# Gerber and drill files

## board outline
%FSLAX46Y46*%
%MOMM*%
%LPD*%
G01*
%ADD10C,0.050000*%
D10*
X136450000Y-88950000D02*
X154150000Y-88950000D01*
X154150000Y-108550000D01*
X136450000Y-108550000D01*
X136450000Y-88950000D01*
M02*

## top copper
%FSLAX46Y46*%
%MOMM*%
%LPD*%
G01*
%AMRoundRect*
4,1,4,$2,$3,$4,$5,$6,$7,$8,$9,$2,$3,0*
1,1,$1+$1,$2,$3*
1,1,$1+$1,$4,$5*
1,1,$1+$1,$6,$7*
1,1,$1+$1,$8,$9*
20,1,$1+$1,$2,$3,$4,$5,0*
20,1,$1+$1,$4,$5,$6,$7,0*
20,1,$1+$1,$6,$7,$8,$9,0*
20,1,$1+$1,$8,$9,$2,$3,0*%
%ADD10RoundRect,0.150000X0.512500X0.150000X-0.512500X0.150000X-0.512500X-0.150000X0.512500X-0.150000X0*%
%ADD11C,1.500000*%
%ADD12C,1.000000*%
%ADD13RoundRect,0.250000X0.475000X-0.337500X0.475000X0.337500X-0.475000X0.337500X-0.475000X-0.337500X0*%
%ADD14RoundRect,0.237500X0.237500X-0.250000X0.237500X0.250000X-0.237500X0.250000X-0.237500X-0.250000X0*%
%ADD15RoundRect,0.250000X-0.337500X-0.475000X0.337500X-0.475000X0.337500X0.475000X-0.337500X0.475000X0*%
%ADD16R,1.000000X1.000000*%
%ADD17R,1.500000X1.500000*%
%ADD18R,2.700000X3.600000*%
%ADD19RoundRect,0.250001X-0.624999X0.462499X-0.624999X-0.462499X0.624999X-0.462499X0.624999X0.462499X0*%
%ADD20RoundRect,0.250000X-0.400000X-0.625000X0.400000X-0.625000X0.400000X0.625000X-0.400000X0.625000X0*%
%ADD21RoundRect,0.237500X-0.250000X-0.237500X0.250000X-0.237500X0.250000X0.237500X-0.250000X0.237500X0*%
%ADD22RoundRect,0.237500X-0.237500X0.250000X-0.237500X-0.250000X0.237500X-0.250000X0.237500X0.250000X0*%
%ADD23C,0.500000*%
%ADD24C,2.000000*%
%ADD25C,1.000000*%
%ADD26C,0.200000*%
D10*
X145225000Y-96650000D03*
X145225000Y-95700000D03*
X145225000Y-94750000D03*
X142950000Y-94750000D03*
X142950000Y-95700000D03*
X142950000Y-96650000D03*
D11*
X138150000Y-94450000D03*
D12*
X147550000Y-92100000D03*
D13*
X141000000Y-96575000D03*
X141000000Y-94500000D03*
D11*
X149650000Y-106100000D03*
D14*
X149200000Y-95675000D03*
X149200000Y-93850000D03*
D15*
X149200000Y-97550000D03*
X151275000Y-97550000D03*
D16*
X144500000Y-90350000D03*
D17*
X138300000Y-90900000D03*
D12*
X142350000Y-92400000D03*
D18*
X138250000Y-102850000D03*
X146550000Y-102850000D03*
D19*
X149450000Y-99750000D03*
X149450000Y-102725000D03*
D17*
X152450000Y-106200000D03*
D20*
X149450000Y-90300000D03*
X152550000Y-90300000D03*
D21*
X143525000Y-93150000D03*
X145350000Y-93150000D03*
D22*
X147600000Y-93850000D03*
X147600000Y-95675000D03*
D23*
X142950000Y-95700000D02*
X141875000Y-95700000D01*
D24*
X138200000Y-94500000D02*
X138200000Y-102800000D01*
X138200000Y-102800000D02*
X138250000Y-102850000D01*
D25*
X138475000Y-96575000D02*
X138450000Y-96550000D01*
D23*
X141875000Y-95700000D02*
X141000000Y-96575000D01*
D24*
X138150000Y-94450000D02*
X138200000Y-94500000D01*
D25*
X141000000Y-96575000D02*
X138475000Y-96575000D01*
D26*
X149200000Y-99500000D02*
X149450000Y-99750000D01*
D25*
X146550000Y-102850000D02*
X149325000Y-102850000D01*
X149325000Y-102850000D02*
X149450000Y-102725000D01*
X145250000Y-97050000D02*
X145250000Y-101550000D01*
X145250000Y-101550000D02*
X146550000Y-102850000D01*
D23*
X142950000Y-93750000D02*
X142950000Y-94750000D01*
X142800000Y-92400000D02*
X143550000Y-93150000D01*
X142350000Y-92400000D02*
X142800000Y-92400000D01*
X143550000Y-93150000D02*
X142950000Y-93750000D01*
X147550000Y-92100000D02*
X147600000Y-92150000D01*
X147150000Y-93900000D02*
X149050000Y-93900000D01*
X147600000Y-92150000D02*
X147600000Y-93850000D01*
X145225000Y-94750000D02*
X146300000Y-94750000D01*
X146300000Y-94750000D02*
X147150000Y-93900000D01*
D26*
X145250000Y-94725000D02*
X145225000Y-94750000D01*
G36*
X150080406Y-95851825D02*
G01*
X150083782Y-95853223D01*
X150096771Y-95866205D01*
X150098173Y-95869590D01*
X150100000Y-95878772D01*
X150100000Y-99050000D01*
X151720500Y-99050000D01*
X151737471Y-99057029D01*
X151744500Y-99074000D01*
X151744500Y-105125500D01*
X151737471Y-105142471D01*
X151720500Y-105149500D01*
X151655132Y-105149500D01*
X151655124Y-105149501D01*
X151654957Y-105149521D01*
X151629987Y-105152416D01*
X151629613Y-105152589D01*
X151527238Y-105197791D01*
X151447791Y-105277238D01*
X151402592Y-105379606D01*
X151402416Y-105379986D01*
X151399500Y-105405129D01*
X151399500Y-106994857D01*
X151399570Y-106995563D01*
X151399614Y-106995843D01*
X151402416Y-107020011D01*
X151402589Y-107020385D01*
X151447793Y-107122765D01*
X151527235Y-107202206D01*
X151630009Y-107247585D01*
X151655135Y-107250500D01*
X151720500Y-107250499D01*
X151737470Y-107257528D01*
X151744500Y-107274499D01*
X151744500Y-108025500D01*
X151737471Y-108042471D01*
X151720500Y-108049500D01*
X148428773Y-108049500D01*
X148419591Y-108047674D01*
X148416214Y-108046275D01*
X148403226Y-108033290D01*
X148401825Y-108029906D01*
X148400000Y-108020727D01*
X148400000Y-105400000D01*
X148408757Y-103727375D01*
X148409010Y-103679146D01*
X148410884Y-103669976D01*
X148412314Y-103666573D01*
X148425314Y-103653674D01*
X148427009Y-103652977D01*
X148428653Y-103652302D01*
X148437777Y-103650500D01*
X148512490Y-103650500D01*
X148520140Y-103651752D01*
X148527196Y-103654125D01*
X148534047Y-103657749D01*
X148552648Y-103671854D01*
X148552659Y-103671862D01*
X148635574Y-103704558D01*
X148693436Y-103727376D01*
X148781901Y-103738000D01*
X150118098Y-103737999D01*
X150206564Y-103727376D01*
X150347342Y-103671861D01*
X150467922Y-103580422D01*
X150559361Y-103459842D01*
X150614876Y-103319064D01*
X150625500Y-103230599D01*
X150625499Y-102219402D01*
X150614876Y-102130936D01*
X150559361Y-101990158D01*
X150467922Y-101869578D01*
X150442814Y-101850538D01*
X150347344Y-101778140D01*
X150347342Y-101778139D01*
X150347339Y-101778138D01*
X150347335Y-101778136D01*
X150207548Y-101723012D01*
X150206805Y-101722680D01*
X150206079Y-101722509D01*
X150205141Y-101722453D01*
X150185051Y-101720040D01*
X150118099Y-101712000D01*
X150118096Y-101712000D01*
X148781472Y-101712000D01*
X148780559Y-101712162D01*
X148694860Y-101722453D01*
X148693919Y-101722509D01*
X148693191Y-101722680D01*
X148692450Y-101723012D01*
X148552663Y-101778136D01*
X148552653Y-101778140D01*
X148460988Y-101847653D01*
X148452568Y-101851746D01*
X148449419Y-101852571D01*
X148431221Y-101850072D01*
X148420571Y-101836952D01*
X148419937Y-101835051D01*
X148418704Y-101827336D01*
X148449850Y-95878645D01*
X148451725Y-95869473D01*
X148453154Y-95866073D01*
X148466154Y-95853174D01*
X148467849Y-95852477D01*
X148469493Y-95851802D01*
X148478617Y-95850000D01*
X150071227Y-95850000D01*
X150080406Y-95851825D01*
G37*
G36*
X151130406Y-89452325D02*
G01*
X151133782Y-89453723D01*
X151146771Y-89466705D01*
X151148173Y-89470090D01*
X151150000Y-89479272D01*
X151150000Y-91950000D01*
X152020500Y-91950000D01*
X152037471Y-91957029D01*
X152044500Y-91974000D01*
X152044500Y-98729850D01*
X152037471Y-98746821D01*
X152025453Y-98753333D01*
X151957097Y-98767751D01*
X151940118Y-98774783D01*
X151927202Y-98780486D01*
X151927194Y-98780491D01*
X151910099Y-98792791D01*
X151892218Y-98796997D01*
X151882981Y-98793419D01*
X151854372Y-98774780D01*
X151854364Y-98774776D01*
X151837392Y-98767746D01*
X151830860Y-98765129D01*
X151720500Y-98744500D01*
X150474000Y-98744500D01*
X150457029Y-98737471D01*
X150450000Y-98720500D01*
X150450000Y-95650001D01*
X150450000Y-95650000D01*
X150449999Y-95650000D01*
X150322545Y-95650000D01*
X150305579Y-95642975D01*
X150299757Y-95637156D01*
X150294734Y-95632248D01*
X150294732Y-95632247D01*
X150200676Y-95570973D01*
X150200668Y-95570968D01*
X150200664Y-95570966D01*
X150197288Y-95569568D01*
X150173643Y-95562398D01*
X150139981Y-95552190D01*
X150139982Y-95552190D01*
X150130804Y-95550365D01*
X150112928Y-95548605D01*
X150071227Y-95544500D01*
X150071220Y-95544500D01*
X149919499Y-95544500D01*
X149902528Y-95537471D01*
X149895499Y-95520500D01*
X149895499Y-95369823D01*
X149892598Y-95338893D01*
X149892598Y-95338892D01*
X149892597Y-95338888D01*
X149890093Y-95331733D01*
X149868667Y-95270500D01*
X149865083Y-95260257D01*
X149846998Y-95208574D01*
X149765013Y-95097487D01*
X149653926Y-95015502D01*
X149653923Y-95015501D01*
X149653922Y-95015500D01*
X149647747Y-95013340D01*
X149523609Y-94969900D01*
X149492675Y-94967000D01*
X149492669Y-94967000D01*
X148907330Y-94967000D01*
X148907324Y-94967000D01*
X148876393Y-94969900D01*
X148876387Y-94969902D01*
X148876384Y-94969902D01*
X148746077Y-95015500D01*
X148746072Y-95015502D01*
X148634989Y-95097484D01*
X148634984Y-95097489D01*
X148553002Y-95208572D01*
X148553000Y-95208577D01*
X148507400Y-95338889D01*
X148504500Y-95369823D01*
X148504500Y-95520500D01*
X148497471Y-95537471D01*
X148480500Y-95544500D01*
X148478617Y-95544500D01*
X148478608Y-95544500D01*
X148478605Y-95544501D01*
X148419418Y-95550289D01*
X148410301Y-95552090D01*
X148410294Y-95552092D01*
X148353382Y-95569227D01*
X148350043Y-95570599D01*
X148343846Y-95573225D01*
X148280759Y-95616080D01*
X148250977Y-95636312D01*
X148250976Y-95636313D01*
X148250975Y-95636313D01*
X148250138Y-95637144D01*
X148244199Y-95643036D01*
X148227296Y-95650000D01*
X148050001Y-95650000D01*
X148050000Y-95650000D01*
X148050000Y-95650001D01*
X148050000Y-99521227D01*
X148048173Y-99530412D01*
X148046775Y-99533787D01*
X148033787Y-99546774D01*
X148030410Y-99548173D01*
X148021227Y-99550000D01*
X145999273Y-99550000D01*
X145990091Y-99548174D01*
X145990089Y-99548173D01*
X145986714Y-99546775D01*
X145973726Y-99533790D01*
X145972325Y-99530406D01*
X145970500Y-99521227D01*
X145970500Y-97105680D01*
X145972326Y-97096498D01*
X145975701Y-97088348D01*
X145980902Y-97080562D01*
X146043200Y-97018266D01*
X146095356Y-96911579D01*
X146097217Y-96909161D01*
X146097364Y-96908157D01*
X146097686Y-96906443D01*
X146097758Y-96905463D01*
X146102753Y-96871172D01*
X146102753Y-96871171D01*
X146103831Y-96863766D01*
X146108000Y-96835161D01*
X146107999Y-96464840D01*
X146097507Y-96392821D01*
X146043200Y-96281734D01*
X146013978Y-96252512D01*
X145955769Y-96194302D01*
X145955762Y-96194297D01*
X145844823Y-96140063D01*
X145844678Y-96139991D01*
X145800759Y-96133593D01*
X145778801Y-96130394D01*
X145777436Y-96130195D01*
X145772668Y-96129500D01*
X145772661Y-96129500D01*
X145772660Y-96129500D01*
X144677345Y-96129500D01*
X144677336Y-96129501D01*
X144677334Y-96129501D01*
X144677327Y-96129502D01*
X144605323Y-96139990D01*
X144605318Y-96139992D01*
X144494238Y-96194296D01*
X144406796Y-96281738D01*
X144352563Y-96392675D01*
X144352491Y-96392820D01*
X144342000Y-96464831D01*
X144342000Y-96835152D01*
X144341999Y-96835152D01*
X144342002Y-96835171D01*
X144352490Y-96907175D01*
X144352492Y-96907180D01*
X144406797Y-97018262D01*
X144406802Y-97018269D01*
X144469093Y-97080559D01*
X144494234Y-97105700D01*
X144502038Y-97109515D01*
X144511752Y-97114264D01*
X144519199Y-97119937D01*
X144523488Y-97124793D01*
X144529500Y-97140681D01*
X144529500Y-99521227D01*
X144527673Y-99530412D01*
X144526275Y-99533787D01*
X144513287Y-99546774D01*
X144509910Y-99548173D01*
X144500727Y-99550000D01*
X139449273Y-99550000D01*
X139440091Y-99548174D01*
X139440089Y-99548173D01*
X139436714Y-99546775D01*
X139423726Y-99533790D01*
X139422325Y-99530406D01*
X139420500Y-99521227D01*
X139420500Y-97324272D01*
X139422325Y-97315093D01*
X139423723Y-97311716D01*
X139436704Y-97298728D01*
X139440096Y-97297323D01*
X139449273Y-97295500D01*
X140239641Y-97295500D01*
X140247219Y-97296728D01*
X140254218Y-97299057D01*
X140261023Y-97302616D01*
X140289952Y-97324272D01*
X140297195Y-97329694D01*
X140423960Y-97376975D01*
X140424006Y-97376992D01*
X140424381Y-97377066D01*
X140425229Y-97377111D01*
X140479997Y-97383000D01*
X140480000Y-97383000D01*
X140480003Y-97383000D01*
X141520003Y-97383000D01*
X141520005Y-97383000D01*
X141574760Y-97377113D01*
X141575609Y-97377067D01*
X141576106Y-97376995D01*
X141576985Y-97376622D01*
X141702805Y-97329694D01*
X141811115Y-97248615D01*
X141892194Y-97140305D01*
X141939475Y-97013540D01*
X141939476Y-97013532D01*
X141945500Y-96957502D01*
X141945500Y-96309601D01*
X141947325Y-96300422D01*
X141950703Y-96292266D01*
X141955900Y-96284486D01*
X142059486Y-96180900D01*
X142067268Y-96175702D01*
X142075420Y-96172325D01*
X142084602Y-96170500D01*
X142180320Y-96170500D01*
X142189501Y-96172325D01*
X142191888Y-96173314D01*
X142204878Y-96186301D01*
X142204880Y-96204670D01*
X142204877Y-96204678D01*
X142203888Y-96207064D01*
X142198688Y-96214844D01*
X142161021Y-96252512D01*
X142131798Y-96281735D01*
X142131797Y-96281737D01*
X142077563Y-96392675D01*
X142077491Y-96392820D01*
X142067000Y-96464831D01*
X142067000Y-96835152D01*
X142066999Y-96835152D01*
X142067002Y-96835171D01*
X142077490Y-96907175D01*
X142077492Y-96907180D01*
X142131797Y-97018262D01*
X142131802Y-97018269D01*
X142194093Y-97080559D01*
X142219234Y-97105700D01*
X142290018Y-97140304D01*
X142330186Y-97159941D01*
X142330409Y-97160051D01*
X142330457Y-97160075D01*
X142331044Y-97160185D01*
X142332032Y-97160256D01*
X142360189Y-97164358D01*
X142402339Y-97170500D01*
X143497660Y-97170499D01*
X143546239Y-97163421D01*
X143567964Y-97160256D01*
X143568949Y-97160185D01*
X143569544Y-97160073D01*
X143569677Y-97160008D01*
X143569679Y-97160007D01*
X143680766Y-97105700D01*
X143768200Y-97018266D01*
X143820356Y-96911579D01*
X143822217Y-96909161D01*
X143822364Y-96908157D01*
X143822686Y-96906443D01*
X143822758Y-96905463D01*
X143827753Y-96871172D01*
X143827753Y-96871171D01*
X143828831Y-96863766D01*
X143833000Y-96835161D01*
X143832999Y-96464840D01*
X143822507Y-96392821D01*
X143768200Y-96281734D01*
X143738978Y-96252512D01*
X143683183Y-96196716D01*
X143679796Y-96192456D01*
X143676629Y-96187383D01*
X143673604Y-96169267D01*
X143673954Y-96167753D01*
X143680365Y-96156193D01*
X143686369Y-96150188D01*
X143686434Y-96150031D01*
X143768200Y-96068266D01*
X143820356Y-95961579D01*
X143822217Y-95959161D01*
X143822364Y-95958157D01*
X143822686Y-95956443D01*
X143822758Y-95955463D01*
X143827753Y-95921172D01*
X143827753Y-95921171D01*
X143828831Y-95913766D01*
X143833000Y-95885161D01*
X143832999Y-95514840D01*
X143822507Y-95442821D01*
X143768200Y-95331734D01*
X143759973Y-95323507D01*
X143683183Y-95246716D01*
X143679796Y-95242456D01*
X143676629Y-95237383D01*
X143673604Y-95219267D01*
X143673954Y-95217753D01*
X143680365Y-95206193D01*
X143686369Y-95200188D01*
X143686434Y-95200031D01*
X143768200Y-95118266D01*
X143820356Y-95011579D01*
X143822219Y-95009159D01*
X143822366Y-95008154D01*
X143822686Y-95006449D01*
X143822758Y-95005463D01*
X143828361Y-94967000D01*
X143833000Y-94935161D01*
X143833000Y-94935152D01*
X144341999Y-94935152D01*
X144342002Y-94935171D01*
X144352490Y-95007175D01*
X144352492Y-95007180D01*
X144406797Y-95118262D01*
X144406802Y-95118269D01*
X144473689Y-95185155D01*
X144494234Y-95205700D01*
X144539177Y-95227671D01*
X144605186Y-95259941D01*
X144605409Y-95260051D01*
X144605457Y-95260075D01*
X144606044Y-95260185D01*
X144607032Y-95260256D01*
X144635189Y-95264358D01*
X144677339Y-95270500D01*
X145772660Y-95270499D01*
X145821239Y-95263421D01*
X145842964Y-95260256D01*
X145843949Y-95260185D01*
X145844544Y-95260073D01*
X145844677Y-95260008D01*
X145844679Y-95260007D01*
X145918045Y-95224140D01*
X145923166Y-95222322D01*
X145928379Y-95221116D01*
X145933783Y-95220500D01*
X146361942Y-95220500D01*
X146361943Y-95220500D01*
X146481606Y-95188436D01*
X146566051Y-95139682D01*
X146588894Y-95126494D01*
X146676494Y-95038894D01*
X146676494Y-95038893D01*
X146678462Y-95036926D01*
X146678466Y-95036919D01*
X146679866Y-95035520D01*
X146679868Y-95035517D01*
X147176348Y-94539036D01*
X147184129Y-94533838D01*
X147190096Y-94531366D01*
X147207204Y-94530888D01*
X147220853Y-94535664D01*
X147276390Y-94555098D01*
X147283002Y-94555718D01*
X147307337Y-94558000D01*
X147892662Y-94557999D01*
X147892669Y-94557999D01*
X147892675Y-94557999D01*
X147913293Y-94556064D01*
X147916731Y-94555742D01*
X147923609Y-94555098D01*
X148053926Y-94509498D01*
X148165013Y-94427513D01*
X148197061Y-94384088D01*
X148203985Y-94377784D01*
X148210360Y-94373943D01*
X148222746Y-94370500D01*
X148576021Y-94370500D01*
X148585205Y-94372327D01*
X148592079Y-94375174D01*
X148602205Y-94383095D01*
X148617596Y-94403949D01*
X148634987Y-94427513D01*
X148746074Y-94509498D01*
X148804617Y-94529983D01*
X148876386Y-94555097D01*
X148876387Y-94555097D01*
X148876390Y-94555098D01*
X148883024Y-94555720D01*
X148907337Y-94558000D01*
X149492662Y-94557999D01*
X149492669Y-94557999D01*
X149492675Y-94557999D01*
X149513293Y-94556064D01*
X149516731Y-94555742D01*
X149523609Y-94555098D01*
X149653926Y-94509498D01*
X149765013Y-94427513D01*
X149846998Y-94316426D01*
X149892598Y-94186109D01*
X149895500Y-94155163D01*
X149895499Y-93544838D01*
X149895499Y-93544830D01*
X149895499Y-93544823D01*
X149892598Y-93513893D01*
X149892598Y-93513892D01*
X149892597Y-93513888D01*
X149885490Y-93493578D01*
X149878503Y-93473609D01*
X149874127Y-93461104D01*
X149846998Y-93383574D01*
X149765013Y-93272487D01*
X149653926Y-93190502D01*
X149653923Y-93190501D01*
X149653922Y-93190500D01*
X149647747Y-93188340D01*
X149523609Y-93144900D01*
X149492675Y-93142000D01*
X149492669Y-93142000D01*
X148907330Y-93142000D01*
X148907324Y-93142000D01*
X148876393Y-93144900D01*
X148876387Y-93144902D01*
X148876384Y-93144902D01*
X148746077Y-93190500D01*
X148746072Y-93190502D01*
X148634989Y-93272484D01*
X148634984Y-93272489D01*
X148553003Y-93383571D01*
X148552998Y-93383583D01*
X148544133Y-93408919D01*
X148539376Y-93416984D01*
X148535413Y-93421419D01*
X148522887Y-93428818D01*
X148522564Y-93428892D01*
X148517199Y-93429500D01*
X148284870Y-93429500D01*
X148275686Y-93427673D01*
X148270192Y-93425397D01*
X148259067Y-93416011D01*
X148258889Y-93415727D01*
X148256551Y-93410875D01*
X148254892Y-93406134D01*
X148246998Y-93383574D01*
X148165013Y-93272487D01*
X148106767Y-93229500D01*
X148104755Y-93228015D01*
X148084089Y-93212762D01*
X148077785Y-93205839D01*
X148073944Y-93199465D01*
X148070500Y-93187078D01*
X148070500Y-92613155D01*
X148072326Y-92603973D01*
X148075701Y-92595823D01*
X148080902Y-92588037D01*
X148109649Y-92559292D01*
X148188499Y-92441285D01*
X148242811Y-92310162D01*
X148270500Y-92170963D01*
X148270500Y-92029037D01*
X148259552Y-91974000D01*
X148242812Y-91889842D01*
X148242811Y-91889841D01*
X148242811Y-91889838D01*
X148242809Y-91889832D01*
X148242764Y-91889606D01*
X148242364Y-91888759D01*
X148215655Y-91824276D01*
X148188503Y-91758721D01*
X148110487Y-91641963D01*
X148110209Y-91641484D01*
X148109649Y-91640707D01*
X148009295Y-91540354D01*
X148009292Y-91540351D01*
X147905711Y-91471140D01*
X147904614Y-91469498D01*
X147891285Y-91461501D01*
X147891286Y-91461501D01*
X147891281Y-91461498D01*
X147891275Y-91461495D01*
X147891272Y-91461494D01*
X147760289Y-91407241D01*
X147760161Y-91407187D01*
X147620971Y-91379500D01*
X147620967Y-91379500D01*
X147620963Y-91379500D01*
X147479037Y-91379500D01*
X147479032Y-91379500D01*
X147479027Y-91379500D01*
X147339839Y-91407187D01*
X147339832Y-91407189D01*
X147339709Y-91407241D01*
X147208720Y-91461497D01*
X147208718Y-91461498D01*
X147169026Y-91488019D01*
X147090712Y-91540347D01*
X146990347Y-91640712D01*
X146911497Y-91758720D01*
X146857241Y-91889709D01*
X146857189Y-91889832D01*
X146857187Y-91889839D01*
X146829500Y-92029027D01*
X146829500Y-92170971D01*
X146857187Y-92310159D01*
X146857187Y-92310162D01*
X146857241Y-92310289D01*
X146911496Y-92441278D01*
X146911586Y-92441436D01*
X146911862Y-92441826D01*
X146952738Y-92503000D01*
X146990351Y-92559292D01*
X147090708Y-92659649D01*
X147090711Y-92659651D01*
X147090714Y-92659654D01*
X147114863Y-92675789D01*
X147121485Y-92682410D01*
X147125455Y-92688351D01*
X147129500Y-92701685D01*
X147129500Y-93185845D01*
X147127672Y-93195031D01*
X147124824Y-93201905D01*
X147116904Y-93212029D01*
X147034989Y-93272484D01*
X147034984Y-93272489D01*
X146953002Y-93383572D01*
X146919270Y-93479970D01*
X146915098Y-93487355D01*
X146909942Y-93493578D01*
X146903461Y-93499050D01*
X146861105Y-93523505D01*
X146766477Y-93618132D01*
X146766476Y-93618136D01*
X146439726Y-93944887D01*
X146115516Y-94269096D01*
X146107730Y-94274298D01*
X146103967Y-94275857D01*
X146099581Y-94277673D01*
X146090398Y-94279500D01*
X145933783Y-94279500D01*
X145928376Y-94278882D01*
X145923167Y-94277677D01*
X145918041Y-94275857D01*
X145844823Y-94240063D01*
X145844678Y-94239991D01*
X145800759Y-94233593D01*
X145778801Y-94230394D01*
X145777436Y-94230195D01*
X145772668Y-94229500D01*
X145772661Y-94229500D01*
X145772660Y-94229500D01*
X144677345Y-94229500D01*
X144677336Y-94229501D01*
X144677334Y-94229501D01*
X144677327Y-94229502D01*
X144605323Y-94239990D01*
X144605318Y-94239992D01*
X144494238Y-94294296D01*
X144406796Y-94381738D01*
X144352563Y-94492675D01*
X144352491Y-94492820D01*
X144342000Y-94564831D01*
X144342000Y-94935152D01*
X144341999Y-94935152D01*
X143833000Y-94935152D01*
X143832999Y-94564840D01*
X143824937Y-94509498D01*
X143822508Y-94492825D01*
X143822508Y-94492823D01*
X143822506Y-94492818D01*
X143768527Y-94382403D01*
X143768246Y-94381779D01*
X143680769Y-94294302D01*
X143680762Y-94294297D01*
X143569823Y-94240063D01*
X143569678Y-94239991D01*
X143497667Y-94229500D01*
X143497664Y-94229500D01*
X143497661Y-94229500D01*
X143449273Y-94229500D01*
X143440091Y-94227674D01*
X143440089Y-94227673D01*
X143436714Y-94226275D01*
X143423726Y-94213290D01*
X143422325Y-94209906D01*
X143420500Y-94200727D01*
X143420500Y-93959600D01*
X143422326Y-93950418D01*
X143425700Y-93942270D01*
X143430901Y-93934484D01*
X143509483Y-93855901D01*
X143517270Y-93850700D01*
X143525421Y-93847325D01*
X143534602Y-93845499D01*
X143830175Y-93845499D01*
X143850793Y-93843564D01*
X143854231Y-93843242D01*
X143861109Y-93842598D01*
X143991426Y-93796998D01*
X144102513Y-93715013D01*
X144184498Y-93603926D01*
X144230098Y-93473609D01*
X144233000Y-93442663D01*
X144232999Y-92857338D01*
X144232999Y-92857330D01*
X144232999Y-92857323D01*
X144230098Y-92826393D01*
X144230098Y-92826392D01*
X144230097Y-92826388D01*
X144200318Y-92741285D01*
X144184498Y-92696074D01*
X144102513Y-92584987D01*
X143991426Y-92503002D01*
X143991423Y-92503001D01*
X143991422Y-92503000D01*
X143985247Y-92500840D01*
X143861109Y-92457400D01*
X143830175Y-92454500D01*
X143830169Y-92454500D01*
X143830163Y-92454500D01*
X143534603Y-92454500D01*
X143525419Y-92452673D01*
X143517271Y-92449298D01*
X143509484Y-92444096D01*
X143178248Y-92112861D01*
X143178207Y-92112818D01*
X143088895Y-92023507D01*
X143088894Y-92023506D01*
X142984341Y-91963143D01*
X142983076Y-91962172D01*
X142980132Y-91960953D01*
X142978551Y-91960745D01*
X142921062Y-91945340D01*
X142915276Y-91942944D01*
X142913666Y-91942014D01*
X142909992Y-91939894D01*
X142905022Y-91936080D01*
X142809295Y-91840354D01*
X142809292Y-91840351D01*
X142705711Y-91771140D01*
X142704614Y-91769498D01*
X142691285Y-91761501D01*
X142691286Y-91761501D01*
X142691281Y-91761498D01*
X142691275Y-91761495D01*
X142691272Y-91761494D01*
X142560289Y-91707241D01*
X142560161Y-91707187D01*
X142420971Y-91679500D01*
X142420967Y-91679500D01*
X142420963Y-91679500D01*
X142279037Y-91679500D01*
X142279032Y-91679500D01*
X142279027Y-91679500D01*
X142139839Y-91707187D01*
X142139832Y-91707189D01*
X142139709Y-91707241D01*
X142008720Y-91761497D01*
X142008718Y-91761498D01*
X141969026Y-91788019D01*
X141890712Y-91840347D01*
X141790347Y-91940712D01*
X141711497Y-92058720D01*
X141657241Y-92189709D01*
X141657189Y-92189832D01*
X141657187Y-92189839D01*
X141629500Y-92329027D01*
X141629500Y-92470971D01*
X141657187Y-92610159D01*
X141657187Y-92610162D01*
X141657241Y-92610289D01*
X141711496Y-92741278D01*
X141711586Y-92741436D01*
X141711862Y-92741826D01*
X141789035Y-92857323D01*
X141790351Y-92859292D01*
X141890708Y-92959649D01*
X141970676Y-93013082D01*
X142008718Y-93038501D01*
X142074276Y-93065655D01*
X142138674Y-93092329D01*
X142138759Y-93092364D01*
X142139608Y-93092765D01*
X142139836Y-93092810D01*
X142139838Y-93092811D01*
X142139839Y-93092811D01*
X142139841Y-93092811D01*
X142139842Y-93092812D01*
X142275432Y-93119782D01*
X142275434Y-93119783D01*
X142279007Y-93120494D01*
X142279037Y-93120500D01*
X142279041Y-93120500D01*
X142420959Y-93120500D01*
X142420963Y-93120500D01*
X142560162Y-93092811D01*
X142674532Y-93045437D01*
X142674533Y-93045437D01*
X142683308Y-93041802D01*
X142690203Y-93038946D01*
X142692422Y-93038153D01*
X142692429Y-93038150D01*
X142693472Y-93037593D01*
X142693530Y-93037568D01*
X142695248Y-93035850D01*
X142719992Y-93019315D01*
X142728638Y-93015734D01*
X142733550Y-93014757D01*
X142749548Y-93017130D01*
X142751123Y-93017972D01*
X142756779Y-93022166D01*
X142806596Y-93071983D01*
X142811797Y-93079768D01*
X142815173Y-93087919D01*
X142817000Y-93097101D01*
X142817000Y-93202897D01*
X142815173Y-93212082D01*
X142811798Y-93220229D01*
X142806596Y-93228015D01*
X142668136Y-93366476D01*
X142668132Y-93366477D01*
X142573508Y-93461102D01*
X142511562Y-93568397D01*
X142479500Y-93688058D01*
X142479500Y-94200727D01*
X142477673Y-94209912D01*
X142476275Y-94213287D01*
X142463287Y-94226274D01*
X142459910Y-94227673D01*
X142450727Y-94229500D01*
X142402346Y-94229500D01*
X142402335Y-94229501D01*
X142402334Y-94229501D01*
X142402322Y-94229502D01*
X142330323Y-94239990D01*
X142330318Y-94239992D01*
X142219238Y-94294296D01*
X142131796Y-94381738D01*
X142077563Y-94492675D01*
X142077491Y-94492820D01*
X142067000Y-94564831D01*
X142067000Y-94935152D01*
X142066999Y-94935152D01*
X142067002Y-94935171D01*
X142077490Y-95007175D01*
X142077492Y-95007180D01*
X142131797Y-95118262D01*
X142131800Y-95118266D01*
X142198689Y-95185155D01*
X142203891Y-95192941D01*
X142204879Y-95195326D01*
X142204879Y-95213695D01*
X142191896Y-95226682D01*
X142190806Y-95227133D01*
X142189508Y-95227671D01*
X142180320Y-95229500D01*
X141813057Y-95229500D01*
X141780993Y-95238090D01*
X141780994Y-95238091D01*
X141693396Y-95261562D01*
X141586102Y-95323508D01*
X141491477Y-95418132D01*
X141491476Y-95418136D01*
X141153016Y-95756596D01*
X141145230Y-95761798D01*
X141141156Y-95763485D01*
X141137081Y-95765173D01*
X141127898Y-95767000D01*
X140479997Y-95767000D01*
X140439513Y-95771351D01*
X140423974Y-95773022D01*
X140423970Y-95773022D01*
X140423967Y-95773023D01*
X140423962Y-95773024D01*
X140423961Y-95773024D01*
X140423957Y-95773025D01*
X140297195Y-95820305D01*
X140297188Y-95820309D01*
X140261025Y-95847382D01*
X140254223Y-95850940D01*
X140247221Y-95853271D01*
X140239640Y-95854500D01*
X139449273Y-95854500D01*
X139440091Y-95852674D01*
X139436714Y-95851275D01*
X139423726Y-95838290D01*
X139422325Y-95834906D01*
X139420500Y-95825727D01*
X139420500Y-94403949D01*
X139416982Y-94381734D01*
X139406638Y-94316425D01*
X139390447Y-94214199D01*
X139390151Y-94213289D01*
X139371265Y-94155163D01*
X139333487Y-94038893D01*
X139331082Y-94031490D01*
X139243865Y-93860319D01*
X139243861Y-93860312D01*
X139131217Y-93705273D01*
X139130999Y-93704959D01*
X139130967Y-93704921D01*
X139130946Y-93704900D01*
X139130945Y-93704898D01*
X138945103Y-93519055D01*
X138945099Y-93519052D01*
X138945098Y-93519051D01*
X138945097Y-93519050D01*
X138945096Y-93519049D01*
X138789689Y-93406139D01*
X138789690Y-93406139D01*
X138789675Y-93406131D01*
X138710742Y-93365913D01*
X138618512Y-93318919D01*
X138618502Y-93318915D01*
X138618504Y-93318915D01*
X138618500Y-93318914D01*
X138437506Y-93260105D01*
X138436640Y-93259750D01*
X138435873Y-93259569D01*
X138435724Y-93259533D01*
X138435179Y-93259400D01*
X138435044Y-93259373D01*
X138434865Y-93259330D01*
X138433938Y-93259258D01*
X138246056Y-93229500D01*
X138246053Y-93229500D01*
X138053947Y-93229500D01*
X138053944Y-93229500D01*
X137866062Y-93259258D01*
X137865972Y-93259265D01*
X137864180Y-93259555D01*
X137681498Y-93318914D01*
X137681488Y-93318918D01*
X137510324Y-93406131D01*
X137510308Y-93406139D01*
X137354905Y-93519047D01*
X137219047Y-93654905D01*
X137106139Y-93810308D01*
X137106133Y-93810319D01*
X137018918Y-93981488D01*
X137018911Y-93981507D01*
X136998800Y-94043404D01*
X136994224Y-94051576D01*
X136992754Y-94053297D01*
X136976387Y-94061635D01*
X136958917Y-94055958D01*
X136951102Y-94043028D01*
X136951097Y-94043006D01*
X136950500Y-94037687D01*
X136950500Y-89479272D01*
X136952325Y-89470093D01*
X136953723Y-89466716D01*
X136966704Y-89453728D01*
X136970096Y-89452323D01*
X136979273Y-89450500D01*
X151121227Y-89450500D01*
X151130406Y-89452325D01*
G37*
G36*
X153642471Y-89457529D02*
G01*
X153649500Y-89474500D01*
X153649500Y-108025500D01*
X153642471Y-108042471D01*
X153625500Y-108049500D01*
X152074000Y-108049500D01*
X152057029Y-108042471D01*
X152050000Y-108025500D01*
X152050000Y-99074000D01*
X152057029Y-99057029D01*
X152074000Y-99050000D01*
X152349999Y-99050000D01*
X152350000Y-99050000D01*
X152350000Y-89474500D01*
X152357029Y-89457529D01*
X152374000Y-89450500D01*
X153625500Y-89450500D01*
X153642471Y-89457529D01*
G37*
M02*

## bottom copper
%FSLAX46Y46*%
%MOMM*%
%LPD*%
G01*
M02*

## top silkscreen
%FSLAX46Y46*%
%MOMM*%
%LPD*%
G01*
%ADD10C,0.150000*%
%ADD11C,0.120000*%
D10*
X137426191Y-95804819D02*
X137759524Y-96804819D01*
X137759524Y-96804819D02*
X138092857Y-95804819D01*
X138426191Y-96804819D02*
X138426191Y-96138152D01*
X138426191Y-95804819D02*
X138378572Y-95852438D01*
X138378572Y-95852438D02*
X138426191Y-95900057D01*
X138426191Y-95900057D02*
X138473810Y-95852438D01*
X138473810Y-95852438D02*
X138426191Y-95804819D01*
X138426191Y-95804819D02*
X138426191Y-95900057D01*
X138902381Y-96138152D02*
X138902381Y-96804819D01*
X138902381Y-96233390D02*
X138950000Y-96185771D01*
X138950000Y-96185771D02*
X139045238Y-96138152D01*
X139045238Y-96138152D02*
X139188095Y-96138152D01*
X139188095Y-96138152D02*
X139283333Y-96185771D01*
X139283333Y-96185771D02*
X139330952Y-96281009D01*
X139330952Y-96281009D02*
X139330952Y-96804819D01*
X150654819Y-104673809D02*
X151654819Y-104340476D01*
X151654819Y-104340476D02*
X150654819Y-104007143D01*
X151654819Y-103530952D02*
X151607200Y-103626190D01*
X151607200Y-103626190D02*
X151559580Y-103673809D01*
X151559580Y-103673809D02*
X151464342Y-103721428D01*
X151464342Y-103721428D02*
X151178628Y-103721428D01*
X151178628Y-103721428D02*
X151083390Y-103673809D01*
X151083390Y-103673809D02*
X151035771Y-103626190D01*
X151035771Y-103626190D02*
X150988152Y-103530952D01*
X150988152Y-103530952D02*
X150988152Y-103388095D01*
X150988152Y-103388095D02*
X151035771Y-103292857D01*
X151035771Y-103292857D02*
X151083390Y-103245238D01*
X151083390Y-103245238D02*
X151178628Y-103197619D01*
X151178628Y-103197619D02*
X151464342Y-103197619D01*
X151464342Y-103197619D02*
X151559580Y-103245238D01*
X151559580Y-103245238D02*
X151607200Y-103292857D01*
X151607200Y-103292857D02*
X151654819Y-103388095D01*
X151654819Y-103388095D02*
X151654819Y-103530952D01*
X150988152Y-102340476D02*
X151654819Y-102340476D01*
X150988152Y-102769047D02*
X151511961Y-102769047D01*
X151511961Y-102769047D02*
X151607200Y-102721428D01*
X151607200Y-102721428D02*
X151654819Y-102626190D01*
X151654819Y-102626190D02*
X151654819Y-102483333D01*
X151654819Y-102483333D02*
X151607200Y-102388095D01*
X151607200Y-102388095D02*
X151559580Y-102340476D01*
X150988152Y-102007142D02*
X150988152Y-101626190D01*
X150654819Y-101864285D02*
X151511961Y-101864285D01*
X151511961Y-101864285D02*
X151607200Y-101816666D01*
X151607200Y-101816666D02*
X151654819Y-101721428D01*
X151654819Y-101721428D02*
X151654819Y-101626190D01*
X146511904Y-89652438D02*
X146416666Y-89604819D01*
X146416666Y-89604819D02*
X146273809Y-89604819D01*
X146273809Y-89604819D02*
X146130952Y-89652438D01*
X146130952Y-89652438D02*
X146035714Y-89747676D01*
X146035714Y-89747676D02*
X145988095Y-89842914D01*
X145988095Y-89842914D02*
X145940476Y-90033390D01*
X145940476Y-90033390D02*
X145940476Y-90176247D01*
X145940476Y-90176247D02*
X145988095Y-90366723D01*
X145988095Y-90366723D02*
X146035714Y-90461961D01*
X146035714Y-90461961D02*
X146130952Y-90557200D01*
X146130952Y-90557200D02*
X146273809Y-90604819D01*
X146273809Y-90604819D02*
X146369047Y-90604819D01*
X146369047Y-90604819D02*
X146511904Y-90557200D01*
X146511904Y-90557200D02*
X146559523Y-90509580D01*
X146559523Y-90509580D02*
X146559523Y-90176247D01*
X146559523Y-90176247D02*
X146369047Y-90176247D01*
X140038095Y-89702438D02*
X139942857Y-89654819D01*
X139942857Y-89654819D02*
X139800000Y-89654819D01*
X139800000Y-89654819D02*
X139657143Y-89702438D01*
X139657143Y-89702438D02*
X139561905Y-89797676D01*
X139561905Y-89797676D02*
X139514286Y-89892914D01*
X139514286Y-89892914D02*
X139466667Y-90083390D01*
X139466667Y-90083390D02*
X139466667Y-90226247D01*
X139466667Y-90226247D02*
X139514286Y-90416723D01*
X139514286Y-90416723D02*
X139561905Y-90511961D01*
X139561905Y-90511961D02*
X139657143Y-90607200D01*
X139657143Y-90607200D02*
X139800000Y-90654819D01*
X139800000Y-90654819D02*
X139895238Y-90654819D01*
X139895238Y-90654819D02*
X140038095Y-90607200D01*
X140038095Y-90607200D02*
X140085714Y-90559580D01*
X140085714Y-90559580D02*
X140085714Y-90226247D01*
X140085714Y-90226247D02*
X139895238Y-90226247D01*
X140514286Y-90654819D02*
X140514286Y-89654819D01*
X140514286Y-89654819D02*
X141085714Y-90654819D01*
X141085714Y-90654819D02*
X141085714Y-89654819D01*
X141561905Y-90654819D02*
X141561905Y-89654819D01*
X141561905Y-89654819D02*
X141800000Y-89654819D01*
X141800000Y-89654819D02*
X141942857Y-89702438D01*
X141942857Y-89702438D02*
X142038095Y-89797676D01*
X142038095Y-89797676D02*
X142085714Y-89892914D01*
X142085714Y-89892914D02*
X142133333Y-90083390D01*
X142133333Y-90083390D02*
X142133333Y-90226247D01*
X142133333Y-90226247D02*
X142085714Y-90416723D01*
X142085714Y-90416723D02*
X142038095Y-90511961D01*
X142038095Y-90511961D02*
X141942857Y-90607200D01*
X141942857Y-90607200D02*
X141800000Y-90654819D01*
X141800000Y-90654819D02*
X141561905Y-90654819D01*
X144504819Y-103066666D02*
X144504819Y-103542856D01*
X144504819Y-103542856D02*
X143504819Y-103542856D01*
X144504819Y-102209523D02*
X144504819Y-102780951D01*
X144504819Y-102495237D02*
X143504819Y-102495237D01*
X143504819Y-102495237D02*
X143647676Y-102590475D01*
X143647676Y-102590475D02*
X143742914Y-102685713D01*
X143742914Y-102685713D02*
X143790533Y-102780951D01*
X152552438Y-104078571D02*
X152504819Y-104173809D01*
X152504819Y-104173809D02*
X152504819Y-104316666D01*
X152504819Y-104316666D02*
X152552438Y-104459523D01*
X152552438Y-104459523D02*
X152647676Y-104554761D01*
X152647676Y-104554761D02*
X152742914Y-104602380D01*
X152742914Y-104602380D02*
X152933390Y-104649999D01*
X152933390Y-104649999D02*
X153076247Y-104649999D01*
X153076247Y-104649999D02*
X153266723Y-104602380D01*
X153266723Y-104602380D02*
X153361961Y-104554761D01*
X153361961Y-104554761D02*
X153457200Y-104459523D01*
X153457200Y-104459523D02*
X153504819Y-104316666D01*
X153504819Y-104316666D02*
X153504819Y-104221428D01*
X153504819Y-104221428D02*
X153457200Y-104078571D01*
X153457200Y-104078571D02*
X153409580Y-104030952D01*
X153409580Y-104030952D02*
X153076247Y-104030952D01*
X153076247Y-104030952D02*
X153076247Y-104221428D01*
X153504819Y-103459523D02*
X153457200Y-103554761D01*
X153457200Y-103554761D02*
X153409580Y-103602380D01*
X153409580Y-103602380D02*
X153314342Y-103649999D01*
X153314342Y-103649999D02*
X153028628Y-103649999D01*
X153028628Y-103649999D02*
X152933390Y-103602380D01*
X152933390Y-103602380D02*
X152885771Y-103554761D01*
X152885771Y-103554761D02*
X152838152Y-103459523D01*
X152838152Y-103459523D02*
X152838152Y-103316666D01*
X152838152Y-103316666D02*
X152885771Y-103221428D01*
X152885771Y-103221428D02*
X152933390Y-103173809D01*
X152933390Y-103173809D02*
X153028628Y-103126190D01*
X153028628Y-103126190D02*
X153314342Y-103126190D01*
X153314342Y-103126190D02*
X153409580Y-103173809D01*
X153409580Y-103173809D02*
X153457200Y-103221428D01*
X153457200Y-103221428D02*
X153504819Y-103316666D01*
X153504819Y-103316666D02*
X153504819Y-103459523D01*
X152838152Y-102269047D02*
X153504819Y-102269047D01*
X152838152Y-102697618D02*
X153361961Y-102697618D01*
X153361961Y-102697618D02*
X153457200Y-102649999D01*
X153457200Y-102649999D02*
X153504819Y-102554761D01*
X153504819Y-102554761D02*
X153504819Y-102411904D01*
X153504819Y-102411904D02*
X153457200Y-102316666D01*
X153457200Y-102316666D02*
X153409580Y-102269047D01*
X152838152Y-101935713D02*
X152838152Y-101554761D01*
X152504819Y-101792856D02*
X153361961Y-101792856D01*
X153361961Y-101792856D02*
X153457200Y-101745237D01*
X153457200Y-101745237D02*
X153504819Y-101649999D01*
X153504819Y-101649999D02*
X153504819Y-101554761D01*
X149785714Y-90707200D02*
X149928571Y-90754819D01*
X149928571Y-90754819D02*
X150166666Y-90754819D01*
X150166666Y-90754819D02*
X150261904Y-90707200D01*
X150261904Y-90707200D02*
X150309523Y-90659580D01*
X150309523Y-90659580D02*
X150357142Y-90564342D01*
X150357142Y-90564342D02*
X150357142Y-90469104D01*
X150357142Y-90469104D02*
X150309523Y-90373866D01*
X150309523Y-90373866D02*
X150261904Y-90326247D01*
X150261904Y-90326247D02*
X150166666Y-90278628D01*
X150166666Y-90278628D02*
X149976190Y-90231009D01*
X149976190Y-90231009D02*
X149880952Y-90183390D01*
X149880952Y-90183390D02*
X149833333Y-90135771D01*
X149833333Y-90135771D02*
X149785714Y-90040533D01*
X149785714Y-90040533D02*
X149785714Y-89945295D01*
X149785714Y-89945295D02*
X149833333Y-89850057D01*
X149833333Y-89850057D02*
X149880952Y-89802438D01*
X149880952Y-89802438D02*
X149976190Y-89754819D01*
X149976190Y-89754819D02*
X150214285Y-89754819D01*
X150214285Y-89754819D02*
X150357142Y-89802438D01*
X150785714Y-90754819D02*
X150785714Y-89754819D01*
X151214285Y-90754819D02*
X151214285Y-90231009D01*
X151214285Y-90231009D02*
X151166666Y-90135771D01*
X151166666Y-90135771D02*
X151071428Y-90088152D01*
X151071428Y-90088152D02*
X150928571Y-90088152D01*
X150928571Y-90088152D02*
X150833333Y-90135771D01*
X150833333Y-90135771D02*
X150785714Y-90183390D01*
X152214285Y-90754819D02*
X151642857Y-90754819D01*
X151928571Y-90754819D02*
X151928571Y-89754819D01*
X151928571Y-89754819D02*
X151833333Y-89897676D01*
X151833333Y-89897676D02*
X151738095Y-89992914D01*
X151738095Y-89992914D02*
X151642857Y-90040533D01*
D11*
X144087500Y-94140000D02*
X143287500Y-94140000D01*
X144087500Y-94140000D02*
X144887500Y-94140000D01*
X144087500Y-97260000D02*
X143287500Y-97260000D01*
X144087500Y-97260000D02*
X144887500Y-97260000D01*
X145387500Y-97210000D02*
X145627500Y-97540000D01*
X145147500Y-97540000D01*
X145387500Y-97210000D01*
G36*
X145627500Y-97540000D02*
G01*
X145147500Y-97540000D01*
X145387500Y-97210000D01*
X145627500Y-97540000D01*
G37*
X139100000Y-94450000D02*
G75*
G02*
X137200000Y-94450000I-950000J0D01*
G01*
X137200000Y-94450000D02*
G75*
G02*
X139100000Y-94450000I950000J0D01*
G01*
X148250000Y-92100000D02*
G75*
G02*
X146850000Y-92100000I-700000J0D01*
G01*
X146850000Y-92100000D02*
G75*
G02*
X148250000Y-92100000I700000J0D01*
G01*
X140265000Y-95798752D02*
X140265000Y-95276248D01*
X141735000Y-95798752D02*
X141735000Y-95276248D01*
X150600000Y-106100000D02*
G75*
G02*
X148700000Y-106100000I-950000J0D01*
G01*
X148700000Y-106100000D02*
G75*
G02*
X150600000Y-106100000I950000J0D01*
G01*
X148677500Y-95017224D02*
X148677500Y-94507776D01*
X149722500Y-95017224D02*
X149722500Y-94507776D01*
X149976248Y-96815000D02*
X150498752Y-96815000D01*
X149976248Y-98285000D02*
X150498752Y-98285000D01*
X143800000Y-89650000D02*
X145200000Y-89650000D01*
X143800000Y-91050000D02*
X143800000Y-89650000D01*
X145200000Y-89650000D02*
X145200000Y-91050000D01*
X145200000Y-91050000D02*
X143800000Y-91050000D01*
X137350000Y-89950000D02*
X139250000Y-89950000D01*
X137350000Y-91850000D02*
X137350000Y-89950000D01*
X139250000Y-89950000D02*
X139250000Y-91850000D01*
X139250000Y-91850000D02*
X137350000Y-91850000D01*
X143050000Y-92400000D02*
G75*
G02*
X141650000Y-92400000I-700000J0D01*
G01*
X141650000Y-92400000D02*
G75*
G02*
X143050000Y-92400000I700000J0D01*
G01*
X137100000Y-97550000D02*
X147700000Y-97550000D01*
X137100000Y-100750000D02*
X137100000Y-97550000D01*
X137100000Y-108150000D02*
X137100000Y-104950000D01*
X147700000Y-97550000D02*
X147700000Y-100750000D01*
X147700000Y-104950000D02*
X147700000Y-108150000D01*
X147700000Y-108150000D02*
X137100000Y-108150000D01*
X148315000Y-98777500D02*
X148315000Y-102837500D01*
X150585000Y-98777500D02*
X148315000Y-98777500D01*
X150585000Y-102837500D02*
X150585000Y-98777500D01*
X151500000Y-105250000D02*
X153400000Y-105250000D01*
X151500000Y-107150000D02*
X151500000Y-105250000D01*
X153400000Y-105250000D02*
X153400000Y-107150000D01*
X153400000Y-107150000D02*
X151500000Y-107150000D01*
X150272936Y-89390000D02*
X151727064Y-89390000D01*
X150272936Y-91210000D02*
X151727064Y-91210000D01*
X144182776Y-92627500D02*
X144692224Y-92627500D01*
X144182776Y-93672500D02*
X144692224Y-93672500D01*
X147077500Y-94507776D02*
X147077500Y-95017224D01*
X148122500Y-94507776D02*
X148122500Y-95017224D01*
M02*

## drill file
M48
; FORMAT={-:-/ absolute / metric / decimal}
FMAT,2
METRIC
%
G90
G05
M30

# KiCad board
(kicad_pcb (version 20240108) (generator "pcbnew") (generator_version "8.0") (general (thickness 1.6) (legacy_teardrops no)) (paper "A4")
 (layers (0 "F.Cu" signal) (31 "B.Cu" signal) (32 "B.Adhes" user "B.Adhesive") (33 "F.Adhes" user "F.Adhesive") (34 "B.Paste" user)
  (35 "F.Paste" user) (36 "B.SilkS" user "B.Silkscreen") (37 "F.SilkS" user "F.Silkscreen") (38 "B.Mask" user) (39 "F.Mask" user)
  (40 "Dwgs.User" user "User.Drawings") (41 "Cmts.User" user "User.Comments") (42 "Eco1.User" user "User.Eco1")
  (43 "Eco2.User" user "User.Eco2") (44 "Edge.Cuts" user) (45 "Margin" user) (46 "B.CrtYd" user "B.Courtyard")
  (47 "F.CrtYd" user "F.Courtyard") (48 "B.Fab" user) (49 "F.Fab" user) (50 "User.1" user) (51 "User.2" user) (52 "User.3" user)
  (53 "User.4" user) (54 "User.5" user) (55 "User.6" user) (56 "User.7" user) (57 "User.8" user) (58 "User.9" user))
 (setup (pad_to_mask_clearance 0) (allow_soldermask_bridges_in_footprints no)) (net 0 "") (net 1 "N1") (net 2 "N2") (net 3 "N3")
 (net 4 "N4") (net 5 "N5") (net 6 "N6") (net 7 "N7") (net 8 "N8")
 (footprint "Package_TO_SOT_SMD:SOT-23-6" (layer "F.Cu") (at 144.0875 95.7 180)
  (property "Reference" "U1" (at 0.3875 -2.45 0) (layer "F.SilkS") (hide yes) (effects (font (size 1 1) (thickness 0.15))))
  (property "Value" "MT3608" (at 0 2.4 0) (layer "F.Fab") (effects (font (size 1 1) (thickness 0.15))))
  (fp_line (start 0 1.56) (end 0.8 1.56) (stroke (width 0.12) (type solid)) (layer "F.SilkS"))
  (fp_line (start 0 1.56) (end -0.8 1.56) (stroke (width 0.12) (type solid)) (layer "F.SilkS"))
  (fp_line (start 0 -1.56) (end 0.8 -1.56) (stroke (width 0.12) (type solid)) (layer "F.SilkS"))
  (fp_line (start 0 -1.56) (end -0.8 -1.56) (stroke (width 0.12) (type solid)) (layer "F.SilkS"))
  (fp_poly
   (pts (xy -1.3 -1.51) (xy -1.54 -1.84) (xy -1.06 -1.84) (xy -1.3 -1.51)) (stroke (width 0.12) (type solid)) (fill solid) (layer "F.SilkS"))
  (pad "1" smd roundrect (at -1.1375 -0.95 180) (size 1.325 0.6) (layers "F.Cu" "F.Paste" "F.Mask") (roundrect_rratio 0.25) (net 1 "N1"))
  (pad "2" smd roundrect (at -1.1375 0 180) (size 1.325 0.6) (layers "F.Cu" "F.Paste" "F.Mask") (roundrect_rratio 0.25) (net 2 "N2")
   (zone_connect 2))
  (pad "3" smd roundrect (at -1.1375 0.95 180) (size 1.325 0.6) (layers "F.Cu" "F.Paste" "F.Mask") (roundrect_rratio 0.25) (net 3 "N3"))
  (pad "4" smd roundrect (at 1.1375 0.95 180) (size 1.325 0.6) (layers "F.Cu" "F.Paste" "F.Mask") (roundrect_rratio 0.25) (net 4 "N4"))
  (pad "5" smd roundrect (at 1.1375 0 180) (size 1.325 0.6) (layers "F.Cu" "F.Paste" "F.Mask") (roundrect_rratio 0.25) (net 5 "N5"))
  (pad "6" smd roundrect (at 1.1375 -0.95 180) (size 1.325 0.6) (layers "F.Cu" "F.Paste" "F.Mask") (roundrect_rratio 0.25) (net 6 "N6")))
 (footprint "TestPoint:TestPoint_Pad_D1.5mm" (layer "F.Cu") (at 138.15 94.45)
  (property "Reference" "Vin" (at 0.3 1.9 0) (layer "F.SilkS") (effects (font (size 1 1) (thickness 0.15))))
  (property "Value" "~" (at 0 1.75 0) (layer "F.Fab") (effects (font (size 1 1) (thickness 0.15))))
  (fp_circle (center 0 0) (end 0 0.95) (stroke (width 0.12) (type solid)) (fill none) (layer "F.SilkS"))
  (pad "1" smd circle (at 0 0) (size 1.5 1.5) (layers "F.Cu" "F.Mask") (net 5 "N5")))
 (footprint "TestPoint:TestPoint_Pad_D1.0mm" (layer "F.Cu") (at 147.55 92.1)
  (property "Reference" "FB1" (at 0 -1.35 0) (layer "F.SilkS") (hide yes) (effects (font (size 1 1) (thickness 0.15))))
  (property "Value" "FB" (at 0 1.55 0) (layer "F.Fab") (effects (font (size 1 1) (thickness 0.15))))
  (fp_circle (center 0 0) (end 0 0.7) (stroke (width 0.12) (type solid)) (fill none) (layer "F.SilkS"))
  (pad "1" smd circle (at 0 0) (size 1 1) (layers "F.Cu" "F.Mask") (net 3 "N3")))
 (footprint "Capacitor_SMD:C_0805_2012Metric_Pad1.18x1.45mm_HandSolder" (layer "F.Cu") (at 141 95.5375 90)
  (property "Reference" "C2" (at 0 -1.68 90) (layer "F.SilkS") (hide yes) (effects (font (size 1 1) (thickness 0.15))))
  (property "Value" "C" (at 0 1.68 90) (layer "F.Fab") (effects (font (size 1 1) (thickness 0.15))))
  (fp_line (start -0.261252 -0.735) (end 0.261252 -0.735) (stroke (width 0.12) (type solid)) (layer "F.SilkS"))
  (fp_line (start -0.261252 0.735) (end 0.261252 0.735) (stroke (width 0.12) (type solid)) (layer "F.SilkS"))
  (pad "1" smd roundrect (at -1.0375 0 90) (size 1.175 1.45) (layers "F.Cu" "F.Paste" "F.Mask") (roundrect_rratio 0.212766) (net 5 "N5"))
  (pad "2" smd roundrect (at 1.0375 0 90) (size 1.175 1.45) (layers "F.Cu" "F.Paste" "F.Mask") (roundrect_rratio 0.212766) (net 2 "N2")
   (zone_connect 2)))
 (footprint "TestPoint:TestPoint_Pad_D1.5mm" (layer "F.Cu") (at 149.65 106.1)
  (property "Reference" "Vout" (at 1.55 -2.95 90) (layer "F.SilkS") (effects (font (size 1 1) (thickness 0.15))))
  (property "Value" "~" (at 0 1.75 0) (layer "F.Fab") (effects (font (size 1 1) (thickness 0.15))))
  (fp_circle (center 0 0) (end 0 0.95) (stroke (width 0.12) (type solid)) (fill none) (layer "F.SilkS"))
  (pad "1" smd circle (at 0 0) (size 1.5 1.5) (layers "F.Cu" "F.Mask") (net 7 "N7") (zone_connect 2)))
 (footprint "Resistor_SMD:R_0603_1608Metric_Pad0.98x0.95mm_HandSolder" (layer "F.Cu") (at 149.2 94.7625 90)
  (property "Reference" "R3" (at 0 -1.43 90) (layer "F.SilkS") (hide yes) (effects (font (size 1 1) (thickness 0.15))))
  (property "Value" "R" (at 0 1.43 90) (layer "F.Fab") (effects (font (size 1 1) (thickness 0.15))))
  (fp_line (start -0.254724 -0.5225) (end 0.254724 -0.5225) (stroke (width 0.12) (type solid)) (layer "F.SilkS"))
  (fp_line (start -0.254724 0.5225) (end 0.254724 0.5225) (stroke (width 0.12) (type solid)) (layer "F.SilkS"))
  (pad "1" smd roundrect (at -0.9125 0 90) (size 0.975 0.95) (layers "F.Cu" "F.Paste" "F.Mask") (roundrect_rratio 0.25) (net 7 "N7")
   (zone_connect 2))
  (pad "2" smd roundrect (at 0.9125 0 90) (size 0.975 0.95) (layers "F.Cu" "F.Paste" "F.Mask") (roundrect_rratio 0.25) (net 3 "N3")))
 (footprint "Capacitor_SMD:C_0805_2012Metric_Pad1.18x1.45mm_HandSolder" (layer "F.Cu") (at 150.2375 97.55)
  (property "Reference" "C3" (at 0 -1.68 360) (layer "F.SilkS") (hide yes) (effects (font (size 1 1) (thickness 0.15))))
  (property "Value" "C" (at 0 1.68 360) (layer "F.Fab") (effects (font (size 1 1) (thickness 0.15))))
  (fp_line (start -0.261252 -0.735) (end 0.261252 -0.735) (stroke (width 0.12) (type solid)) (layer "F.SilkS"))
  (fp_line (start -0.261252 0.735) (end 0.261252 0.735) (stroke (width 0.12) (type solid)) (layer "F.SilkS"))
  (pad "1" smd roundrect (at -1.0375 0) (size 1.175 1.45) (layers "F.Cu" "F.Paste" "F.Mask") (roundrect_rratio 0.212766) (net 7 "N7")
   (zone_connect 2))
  (pad "2" smd roundrect (at 1.0375 0) (size 1.175 1.45) (layers "F.Cu" "F.Paste" "F.Mask") (roundrect_rratio 0.212766) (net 2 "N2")
   (zone_connect 2)))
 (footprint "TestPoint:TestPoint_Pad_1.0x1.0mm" (layer "F.Cu") (at 144.5 90.35)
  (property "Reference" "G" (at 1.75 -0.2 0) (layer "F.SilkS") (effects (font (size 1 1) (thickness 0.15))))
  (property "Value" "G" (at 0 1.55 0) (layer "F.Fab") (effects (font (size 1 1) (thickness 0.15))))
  (fp_line (start -0.7 -0.7) (end 0.7 -0.7) (stroke (width 0.12) (type solid)) (layer "F.SilkS"))
  (fp_line (start -0.7 0.7) (end -0.7 -0.7) (stroke (width 0.12) (type solid)) (layer "F.SilkS"))
  (fp_line (start 0.7 -0.7) (end 0.7 0.7) (stroke (width 0.12) (type solid)) (layer "F.SilkS"))
  (fp_line (start 0.7 0.7) (end -0.7 0.7) (stroke (width 0.12) (type solid)) (layer "F.SilkS"))
  (pad "1" smd rect (at 0 0) (size 1 1) (layers "F.Cu" "F.Mask") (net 2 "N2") (zone_connect 2)))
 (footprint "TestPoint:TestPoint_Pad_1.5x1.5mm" (layer "F.Cu") (at 138.3 90.9)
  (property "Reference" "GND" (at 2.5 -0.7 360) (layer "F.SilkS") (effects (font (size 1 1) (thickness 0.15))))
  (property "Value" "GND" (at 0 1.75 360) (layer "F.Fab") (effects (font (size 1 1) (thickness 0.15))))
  (fp_line (start -0.95 -0.95) (end 0.95 -0.95) (stroke (width 0.12) (type solid)) (layer "F.SilkS"))
  (fp_line (start -0.95 0.95) (end -0.95 -0.95) (stroke (width 0.12) (type solid)) (layer "F.SilkS"))
  (fp_line (start 0.95 -0.95) (end 0.95 0.95) (stroke (width 0.12) (type solid)) (layer "F.SilkS"))
  (fp_line (start 0.95 0.95) (end -0.95 0.95) (stroke (width 0.12) (type solid)) (layer "F.SilkS"))
  (pad "1" smd rect (at 0 0) (size 1.5 1.5) (layers "F.Cu" "F.Mask") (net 2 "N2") (zone_connect 2)))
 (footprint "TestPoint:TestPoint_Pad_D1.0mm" (layer "F.Cu") (at 142.35 92.4 180)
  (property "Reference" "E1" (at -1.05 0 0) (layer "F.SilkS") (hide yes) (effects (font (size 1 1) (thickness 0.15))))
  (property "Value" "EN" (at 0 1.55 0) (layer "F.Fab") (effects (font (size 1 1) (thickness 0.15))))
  (fp_circle (center 0 0) (end 0 0.7) (stroke (width 0.12) (type solid)) (fill none) (layer "F.SilkS"))
  (pad "1" smd circle (at 0 0 180) (size 1 1) (layers "F.Cu" "F.Mask") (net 4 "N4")))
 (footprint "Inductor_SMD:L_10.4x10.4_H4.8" (layer "F.Cu") (at 142.4 102.85)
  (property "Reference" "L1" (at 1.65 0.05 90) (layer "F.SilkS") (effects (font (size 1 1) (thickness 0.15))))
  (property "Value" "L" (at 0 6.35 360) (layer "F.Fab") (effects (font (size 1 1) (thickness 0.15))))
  (fp_line (start -5.3 -5.3) (end 5.3 -5.3) (stroke (width 0.12) (type solid)) (layer "F.SilkS"))
  (fp_line (start -5.3 -2.1) (end -5.3 -5.3) (stroke (width 0.12) (type solid)) (layer "F.SilkS"))
  (fp_line (start -5.3 5.3) (end -5.3 2.1) (stroke (width 0.12) (type solid)) (layer "F.SilkS"))
  (fp_line (start 5.3 -5.3) (end 5.3 -2.1) (stroke (width 0.12) (type solid)) (layer "F.SilkS"))
  (fp_line (start 5.3 2.1) (end 5.3 5.3) (stroke (width 0.12) (type solid)) (layer "F.SilkS"))
  (fp_line (start 5.3 5.3) (end -5.3 5.3) (stroke (width 0.12) (type solid)) (layer "F.SilkS"))
  (pad "1" smd rect (at -4.15 0) (size 2.7 3.6) (layers "F.Cu" "F.Paste" "F.Mask") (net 5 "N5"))
  (pad "2" smd rect (at 4.15 0) (size 2.7 3.6) (layers "F.Cu" "F.Paste" "F.Mask") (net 1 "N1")))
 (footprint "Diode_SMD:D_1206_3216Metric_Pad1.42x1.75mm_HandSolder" (layer "F.Cu") (at 149.45 101.2375 -90)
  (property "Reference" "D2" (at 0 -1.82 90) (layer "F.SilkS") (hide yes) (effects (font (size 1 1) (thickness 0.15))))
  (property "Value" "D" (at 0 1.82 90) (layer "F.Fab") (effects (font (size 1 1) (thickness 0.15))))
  (fp_line (start -2.46 1.135) (end 1.6 1.135) (stroke (width 0.12) (type solid)) (layer "F.SilkS"))
  (fp_line (start -2.46 -1.135) (end -2.46 1.135) (stroke (width 0.12) (type solid)) (layer "F.SilkS"))
  (fp_line (start 1.6 -1.135) (end -2.46 -1.135) (stroke (width 0.12) (type solid)) (layer "F.SilkS"))
  (pad "1" smd roundrect (at -1.4875 0 270) (size 1.425 1.75) (layers "F.Cu" "F.Paste" "F.Mask") (roundrect_rratio 0.175439) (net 7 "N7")
   (zone_connect 2))
  (pad "2" smd roundrect (at 1.4875 0 270) (size 1.425 1.75) (layers "F.Cu" "F.Paste" "F.Mask") (roundrect_rratio 0.175439) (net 1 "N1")))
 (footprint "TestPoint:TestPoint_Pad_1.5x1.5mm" (layer "F.Cu") (at 152.45 106.2)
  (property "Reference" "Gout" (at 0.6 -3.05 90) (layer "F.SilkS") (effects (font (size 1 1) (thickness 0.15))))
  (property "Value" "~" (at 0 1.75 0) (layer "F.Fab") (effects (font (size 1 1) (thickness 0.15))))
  (fp_line (start -0.95 -0.95) (end 0.95 -0.95) (stroke (width 0.12) (type solid)) (layer "F.SilkS"))
  (fp_line (start -0.95 0.95) (end -0.95 -0.95) (stroke (width 0.12) (type solid)) (layer "F.SilkS"))
  (fp_line (start 0.95 -0.95) (end 0.95 0.95) (stroke (width 0.12) (type solid)) (layer "F.SilkS"))
  (fp_line (start 0.95 0.95) (end -0.95 0.95) (stroke (width 0.12) (type solid)) (layer "F.SilkS"))
  (pad "1" smd rect (at 0 0) (size 1.5 1.5) (layers "F.Cu" "F.Mask") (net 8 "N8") (zone_connect 2)))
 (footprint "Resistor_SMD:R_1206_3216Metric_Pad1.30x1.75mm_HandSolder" (layer "F.Cu") (at 151 90.3)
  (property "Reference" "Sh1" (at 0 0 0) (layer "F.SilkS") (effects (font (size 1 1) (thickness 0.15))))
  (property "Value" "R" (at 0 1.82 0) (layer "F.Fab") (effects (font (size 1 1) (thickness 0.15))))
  (fp_line (start -0.727064 -0.91) (end 0.727064 -0.91) (stroke (width 0.12) (type solid)) (layer "F.SilkS"))
  (fp_line (start -0.727064 0.91) (end 0.727064 0.91) (stroke (width 0.12) (type solid)) (layer "F.SilkS"))
  (pad "1" smd roundrect (at -1.55 0) (size 1.3 1.75) (layers "F.Cu" "F.Paste" "F.Mask") (roundrect_rratio 0.192308) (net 2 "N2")
   (zone_connect 2))
  (pad "2" smd roundrect (at 1.55 0) (size 1.3 1.75) (layers "F.Cu" "F.Paste" "F.Mask") (roundrect_rratio 0.192308) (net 8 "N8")
   (zone_connect 2)))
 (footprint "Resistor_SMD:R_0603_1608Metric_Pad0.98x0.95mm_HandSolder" (layer "F.Cu") (at 144.4375 93.15)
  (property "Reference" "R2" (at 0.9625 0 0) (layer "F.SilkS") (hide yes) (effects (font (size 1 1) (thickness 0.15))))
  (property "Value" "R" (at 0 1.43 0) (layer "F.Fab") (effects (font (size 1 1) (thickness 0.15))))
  (fp_line (start -0.254724 -0.5225) (end 0.254724 -0.5225) (stroke (width 0.12) (type solid)) (layer "F.SilkS"))
  (fp_line (start -0.254724 0.5225) (end 0.254724 0.5225) (stroke (width 0.12) (type solid)) (layer "F.SilkS"))
  (pad "1" smd roundrect (at -0.9125 0) (size 0.975 0.95) (layers "F.Cu" "F.Paste" "F.Mask") (roundrect_rratio 0.25) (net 4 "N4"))
  (pad "2" smd roundrect (at 0.9125 0) (size 0.975 0.95) (layers "F.Cu" "F.Paste" "F.Mask") (roundrect_rratio 0.25) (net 2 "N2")
   (zone_connect 2)))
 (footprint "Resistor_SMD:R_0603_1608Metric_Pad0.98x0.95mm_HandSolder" (layer "F.Cu") (at 147.6 94.7625 -90)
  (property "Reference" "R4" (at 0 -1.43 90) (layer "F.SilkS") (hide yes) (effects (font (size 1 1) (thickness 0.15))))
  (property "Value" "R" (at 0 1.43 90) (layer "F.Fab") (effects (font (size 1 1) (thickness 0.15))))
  (fp_line (start -0.254724 0.5225) (end 0.254724 0.5225) (stroke (width 0.12) (type solid)) (layer "F.SilkS"))
  (fp_line (start -0.254724 -0.5225) (end 0.254724 -0.5225) (stroke (width 0.12) (type solid)) (layer "F.SilkS"))
  (pad "1" smd roundrect (at -0.9125 0 270) (size 0.975 0.95) (layers "F.Cu" "F.Paste" "F.Mask") (roundrect_rratio 0.25) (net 3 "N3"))
  (pad "2" smd roundrect (at 0.9125 0 270) (size 0.975 0.95) (layers "F.Cu" "F.Paste" "F.Mask") (roundrect_rratio 0.25) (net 2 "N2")
   (zone_connect 2)))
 (gr_rect (start 136.45 88.95) (end 154.15 108.55) (stroke (width 0.05) (type default)) (fill none) (layer "Edge.Cuts"))
 (segment (start 142.95 95.7) (end 141.875 95.7) (width 0.5) (layer "F.Cu") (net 5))
 (segment (start 138.2 94.5) (end 138.2 102.8) (width 2) (layer "F.Cu") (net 5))
 (segment (start 138.2 102.8) (end 138.25 102.85) (width 2) (layer "F.Cu") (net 5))
 (segment (start 138.475 96.575) (end 138.45 96.55) (width 1) (layer "F.Cu") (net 5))
 (segment (start 141.875 95.7) (end 141 96.575) (width 0.5) (layer "F.Cu") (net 5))
 (segment (start 138.15 94.45) (end 138.2 94.5) (width 2) (layer "F.Cu") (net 5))
 (segment (start 141 96.575) (end 138.475 96.575) (width 1) (layer "F.Cu") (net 5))
 (segment (start 149.2 99.5) (end 149.45 99.75) (width 0.2) (layer "F.Cu") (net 7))
 (segment (start 146.55 102.85) (end 149.325 102.85) (width 1) (layer "F.Cu") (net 1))
 (segment (start 149.325 102.85) (end 149.45 102.725) (width 1) (layer "F.Cu") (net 1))
 (segment (start 145.25 97.05) (end 145.25 101.55) (width 1) (layer "F.Cu") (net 1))
 (segment (start 145.25 101.55) (end 146.55 102.85) (width 1) (layer "F.Cu") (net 1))
 (segment (start 142.95 93.75) (end 142.95 94.75) (width 0.5) (layer "F.Cu") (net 4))
 (segment (start 142.8 92.4) (end 143.55 93.15) (width 0.5) (layer "F.Cu") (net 4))
 (segment (start 142.35 92.4) (end 142.8 92.4) (width 0.5) (layer "F.Cu") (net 4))
 (segment (start 143.55 93.15) (end 142.95 93.75) (width 0.5) (layer "F.Cu") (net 4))
 (segment (start 147.55 92.1) (end 147.6 92.15) (width 0.5) (layer "F.Cu") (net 3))
 (segment (start 147.15 93.9) (end 149.05 93.9) (width 0.5) (layer "F.Cu") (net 3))
 (segment (start 147.6 92.15) (end 147.6 93.85) (width 0.5) (layer "F.Cu") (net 3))
 (segment (start 145.225 94.75) (end 146.3 94.75) (width 0.5) (layer "F.Cu") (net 3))
 (segment (start 146.3 94.75) (end 147.15 93.9) (width 0.5) (layer "F.Cu") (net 3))
 (segment (start 145.25 94.725) (end 145.225 94.75) (width 0.2) (layer "F.Cu") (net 3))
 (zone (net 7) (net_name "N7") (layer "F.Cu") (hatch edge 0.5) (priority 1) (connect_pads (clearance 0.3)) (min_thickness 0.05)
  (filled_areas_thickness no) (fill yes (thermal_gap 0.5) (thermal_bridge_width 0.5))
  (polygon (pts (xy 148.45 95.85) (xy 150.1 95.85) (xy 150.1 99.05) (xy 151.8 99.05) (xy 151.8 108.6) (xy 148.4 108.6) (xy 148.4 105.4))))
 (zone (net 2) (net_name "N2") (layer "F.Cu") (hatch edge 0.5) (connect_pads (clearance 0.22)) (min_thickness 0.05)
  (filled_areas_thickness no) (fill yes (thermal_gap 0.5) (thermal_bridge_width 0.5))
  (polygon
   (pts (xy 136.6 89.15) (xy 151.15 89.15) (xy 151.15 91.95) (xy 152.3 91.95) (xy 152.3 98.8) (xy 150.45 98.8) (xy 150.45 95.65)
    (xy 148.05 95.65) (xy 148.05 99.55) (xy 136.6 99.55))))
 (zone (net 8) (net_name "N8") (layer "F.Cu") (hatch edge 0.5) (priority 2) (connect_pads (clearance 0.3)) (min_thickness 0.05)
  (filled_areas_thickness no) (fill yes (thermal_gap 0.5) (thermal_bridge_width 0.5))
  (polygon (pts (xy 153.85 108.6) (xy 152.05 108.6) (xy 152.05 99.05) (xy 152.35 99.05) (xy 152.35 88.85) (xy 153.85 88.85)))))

